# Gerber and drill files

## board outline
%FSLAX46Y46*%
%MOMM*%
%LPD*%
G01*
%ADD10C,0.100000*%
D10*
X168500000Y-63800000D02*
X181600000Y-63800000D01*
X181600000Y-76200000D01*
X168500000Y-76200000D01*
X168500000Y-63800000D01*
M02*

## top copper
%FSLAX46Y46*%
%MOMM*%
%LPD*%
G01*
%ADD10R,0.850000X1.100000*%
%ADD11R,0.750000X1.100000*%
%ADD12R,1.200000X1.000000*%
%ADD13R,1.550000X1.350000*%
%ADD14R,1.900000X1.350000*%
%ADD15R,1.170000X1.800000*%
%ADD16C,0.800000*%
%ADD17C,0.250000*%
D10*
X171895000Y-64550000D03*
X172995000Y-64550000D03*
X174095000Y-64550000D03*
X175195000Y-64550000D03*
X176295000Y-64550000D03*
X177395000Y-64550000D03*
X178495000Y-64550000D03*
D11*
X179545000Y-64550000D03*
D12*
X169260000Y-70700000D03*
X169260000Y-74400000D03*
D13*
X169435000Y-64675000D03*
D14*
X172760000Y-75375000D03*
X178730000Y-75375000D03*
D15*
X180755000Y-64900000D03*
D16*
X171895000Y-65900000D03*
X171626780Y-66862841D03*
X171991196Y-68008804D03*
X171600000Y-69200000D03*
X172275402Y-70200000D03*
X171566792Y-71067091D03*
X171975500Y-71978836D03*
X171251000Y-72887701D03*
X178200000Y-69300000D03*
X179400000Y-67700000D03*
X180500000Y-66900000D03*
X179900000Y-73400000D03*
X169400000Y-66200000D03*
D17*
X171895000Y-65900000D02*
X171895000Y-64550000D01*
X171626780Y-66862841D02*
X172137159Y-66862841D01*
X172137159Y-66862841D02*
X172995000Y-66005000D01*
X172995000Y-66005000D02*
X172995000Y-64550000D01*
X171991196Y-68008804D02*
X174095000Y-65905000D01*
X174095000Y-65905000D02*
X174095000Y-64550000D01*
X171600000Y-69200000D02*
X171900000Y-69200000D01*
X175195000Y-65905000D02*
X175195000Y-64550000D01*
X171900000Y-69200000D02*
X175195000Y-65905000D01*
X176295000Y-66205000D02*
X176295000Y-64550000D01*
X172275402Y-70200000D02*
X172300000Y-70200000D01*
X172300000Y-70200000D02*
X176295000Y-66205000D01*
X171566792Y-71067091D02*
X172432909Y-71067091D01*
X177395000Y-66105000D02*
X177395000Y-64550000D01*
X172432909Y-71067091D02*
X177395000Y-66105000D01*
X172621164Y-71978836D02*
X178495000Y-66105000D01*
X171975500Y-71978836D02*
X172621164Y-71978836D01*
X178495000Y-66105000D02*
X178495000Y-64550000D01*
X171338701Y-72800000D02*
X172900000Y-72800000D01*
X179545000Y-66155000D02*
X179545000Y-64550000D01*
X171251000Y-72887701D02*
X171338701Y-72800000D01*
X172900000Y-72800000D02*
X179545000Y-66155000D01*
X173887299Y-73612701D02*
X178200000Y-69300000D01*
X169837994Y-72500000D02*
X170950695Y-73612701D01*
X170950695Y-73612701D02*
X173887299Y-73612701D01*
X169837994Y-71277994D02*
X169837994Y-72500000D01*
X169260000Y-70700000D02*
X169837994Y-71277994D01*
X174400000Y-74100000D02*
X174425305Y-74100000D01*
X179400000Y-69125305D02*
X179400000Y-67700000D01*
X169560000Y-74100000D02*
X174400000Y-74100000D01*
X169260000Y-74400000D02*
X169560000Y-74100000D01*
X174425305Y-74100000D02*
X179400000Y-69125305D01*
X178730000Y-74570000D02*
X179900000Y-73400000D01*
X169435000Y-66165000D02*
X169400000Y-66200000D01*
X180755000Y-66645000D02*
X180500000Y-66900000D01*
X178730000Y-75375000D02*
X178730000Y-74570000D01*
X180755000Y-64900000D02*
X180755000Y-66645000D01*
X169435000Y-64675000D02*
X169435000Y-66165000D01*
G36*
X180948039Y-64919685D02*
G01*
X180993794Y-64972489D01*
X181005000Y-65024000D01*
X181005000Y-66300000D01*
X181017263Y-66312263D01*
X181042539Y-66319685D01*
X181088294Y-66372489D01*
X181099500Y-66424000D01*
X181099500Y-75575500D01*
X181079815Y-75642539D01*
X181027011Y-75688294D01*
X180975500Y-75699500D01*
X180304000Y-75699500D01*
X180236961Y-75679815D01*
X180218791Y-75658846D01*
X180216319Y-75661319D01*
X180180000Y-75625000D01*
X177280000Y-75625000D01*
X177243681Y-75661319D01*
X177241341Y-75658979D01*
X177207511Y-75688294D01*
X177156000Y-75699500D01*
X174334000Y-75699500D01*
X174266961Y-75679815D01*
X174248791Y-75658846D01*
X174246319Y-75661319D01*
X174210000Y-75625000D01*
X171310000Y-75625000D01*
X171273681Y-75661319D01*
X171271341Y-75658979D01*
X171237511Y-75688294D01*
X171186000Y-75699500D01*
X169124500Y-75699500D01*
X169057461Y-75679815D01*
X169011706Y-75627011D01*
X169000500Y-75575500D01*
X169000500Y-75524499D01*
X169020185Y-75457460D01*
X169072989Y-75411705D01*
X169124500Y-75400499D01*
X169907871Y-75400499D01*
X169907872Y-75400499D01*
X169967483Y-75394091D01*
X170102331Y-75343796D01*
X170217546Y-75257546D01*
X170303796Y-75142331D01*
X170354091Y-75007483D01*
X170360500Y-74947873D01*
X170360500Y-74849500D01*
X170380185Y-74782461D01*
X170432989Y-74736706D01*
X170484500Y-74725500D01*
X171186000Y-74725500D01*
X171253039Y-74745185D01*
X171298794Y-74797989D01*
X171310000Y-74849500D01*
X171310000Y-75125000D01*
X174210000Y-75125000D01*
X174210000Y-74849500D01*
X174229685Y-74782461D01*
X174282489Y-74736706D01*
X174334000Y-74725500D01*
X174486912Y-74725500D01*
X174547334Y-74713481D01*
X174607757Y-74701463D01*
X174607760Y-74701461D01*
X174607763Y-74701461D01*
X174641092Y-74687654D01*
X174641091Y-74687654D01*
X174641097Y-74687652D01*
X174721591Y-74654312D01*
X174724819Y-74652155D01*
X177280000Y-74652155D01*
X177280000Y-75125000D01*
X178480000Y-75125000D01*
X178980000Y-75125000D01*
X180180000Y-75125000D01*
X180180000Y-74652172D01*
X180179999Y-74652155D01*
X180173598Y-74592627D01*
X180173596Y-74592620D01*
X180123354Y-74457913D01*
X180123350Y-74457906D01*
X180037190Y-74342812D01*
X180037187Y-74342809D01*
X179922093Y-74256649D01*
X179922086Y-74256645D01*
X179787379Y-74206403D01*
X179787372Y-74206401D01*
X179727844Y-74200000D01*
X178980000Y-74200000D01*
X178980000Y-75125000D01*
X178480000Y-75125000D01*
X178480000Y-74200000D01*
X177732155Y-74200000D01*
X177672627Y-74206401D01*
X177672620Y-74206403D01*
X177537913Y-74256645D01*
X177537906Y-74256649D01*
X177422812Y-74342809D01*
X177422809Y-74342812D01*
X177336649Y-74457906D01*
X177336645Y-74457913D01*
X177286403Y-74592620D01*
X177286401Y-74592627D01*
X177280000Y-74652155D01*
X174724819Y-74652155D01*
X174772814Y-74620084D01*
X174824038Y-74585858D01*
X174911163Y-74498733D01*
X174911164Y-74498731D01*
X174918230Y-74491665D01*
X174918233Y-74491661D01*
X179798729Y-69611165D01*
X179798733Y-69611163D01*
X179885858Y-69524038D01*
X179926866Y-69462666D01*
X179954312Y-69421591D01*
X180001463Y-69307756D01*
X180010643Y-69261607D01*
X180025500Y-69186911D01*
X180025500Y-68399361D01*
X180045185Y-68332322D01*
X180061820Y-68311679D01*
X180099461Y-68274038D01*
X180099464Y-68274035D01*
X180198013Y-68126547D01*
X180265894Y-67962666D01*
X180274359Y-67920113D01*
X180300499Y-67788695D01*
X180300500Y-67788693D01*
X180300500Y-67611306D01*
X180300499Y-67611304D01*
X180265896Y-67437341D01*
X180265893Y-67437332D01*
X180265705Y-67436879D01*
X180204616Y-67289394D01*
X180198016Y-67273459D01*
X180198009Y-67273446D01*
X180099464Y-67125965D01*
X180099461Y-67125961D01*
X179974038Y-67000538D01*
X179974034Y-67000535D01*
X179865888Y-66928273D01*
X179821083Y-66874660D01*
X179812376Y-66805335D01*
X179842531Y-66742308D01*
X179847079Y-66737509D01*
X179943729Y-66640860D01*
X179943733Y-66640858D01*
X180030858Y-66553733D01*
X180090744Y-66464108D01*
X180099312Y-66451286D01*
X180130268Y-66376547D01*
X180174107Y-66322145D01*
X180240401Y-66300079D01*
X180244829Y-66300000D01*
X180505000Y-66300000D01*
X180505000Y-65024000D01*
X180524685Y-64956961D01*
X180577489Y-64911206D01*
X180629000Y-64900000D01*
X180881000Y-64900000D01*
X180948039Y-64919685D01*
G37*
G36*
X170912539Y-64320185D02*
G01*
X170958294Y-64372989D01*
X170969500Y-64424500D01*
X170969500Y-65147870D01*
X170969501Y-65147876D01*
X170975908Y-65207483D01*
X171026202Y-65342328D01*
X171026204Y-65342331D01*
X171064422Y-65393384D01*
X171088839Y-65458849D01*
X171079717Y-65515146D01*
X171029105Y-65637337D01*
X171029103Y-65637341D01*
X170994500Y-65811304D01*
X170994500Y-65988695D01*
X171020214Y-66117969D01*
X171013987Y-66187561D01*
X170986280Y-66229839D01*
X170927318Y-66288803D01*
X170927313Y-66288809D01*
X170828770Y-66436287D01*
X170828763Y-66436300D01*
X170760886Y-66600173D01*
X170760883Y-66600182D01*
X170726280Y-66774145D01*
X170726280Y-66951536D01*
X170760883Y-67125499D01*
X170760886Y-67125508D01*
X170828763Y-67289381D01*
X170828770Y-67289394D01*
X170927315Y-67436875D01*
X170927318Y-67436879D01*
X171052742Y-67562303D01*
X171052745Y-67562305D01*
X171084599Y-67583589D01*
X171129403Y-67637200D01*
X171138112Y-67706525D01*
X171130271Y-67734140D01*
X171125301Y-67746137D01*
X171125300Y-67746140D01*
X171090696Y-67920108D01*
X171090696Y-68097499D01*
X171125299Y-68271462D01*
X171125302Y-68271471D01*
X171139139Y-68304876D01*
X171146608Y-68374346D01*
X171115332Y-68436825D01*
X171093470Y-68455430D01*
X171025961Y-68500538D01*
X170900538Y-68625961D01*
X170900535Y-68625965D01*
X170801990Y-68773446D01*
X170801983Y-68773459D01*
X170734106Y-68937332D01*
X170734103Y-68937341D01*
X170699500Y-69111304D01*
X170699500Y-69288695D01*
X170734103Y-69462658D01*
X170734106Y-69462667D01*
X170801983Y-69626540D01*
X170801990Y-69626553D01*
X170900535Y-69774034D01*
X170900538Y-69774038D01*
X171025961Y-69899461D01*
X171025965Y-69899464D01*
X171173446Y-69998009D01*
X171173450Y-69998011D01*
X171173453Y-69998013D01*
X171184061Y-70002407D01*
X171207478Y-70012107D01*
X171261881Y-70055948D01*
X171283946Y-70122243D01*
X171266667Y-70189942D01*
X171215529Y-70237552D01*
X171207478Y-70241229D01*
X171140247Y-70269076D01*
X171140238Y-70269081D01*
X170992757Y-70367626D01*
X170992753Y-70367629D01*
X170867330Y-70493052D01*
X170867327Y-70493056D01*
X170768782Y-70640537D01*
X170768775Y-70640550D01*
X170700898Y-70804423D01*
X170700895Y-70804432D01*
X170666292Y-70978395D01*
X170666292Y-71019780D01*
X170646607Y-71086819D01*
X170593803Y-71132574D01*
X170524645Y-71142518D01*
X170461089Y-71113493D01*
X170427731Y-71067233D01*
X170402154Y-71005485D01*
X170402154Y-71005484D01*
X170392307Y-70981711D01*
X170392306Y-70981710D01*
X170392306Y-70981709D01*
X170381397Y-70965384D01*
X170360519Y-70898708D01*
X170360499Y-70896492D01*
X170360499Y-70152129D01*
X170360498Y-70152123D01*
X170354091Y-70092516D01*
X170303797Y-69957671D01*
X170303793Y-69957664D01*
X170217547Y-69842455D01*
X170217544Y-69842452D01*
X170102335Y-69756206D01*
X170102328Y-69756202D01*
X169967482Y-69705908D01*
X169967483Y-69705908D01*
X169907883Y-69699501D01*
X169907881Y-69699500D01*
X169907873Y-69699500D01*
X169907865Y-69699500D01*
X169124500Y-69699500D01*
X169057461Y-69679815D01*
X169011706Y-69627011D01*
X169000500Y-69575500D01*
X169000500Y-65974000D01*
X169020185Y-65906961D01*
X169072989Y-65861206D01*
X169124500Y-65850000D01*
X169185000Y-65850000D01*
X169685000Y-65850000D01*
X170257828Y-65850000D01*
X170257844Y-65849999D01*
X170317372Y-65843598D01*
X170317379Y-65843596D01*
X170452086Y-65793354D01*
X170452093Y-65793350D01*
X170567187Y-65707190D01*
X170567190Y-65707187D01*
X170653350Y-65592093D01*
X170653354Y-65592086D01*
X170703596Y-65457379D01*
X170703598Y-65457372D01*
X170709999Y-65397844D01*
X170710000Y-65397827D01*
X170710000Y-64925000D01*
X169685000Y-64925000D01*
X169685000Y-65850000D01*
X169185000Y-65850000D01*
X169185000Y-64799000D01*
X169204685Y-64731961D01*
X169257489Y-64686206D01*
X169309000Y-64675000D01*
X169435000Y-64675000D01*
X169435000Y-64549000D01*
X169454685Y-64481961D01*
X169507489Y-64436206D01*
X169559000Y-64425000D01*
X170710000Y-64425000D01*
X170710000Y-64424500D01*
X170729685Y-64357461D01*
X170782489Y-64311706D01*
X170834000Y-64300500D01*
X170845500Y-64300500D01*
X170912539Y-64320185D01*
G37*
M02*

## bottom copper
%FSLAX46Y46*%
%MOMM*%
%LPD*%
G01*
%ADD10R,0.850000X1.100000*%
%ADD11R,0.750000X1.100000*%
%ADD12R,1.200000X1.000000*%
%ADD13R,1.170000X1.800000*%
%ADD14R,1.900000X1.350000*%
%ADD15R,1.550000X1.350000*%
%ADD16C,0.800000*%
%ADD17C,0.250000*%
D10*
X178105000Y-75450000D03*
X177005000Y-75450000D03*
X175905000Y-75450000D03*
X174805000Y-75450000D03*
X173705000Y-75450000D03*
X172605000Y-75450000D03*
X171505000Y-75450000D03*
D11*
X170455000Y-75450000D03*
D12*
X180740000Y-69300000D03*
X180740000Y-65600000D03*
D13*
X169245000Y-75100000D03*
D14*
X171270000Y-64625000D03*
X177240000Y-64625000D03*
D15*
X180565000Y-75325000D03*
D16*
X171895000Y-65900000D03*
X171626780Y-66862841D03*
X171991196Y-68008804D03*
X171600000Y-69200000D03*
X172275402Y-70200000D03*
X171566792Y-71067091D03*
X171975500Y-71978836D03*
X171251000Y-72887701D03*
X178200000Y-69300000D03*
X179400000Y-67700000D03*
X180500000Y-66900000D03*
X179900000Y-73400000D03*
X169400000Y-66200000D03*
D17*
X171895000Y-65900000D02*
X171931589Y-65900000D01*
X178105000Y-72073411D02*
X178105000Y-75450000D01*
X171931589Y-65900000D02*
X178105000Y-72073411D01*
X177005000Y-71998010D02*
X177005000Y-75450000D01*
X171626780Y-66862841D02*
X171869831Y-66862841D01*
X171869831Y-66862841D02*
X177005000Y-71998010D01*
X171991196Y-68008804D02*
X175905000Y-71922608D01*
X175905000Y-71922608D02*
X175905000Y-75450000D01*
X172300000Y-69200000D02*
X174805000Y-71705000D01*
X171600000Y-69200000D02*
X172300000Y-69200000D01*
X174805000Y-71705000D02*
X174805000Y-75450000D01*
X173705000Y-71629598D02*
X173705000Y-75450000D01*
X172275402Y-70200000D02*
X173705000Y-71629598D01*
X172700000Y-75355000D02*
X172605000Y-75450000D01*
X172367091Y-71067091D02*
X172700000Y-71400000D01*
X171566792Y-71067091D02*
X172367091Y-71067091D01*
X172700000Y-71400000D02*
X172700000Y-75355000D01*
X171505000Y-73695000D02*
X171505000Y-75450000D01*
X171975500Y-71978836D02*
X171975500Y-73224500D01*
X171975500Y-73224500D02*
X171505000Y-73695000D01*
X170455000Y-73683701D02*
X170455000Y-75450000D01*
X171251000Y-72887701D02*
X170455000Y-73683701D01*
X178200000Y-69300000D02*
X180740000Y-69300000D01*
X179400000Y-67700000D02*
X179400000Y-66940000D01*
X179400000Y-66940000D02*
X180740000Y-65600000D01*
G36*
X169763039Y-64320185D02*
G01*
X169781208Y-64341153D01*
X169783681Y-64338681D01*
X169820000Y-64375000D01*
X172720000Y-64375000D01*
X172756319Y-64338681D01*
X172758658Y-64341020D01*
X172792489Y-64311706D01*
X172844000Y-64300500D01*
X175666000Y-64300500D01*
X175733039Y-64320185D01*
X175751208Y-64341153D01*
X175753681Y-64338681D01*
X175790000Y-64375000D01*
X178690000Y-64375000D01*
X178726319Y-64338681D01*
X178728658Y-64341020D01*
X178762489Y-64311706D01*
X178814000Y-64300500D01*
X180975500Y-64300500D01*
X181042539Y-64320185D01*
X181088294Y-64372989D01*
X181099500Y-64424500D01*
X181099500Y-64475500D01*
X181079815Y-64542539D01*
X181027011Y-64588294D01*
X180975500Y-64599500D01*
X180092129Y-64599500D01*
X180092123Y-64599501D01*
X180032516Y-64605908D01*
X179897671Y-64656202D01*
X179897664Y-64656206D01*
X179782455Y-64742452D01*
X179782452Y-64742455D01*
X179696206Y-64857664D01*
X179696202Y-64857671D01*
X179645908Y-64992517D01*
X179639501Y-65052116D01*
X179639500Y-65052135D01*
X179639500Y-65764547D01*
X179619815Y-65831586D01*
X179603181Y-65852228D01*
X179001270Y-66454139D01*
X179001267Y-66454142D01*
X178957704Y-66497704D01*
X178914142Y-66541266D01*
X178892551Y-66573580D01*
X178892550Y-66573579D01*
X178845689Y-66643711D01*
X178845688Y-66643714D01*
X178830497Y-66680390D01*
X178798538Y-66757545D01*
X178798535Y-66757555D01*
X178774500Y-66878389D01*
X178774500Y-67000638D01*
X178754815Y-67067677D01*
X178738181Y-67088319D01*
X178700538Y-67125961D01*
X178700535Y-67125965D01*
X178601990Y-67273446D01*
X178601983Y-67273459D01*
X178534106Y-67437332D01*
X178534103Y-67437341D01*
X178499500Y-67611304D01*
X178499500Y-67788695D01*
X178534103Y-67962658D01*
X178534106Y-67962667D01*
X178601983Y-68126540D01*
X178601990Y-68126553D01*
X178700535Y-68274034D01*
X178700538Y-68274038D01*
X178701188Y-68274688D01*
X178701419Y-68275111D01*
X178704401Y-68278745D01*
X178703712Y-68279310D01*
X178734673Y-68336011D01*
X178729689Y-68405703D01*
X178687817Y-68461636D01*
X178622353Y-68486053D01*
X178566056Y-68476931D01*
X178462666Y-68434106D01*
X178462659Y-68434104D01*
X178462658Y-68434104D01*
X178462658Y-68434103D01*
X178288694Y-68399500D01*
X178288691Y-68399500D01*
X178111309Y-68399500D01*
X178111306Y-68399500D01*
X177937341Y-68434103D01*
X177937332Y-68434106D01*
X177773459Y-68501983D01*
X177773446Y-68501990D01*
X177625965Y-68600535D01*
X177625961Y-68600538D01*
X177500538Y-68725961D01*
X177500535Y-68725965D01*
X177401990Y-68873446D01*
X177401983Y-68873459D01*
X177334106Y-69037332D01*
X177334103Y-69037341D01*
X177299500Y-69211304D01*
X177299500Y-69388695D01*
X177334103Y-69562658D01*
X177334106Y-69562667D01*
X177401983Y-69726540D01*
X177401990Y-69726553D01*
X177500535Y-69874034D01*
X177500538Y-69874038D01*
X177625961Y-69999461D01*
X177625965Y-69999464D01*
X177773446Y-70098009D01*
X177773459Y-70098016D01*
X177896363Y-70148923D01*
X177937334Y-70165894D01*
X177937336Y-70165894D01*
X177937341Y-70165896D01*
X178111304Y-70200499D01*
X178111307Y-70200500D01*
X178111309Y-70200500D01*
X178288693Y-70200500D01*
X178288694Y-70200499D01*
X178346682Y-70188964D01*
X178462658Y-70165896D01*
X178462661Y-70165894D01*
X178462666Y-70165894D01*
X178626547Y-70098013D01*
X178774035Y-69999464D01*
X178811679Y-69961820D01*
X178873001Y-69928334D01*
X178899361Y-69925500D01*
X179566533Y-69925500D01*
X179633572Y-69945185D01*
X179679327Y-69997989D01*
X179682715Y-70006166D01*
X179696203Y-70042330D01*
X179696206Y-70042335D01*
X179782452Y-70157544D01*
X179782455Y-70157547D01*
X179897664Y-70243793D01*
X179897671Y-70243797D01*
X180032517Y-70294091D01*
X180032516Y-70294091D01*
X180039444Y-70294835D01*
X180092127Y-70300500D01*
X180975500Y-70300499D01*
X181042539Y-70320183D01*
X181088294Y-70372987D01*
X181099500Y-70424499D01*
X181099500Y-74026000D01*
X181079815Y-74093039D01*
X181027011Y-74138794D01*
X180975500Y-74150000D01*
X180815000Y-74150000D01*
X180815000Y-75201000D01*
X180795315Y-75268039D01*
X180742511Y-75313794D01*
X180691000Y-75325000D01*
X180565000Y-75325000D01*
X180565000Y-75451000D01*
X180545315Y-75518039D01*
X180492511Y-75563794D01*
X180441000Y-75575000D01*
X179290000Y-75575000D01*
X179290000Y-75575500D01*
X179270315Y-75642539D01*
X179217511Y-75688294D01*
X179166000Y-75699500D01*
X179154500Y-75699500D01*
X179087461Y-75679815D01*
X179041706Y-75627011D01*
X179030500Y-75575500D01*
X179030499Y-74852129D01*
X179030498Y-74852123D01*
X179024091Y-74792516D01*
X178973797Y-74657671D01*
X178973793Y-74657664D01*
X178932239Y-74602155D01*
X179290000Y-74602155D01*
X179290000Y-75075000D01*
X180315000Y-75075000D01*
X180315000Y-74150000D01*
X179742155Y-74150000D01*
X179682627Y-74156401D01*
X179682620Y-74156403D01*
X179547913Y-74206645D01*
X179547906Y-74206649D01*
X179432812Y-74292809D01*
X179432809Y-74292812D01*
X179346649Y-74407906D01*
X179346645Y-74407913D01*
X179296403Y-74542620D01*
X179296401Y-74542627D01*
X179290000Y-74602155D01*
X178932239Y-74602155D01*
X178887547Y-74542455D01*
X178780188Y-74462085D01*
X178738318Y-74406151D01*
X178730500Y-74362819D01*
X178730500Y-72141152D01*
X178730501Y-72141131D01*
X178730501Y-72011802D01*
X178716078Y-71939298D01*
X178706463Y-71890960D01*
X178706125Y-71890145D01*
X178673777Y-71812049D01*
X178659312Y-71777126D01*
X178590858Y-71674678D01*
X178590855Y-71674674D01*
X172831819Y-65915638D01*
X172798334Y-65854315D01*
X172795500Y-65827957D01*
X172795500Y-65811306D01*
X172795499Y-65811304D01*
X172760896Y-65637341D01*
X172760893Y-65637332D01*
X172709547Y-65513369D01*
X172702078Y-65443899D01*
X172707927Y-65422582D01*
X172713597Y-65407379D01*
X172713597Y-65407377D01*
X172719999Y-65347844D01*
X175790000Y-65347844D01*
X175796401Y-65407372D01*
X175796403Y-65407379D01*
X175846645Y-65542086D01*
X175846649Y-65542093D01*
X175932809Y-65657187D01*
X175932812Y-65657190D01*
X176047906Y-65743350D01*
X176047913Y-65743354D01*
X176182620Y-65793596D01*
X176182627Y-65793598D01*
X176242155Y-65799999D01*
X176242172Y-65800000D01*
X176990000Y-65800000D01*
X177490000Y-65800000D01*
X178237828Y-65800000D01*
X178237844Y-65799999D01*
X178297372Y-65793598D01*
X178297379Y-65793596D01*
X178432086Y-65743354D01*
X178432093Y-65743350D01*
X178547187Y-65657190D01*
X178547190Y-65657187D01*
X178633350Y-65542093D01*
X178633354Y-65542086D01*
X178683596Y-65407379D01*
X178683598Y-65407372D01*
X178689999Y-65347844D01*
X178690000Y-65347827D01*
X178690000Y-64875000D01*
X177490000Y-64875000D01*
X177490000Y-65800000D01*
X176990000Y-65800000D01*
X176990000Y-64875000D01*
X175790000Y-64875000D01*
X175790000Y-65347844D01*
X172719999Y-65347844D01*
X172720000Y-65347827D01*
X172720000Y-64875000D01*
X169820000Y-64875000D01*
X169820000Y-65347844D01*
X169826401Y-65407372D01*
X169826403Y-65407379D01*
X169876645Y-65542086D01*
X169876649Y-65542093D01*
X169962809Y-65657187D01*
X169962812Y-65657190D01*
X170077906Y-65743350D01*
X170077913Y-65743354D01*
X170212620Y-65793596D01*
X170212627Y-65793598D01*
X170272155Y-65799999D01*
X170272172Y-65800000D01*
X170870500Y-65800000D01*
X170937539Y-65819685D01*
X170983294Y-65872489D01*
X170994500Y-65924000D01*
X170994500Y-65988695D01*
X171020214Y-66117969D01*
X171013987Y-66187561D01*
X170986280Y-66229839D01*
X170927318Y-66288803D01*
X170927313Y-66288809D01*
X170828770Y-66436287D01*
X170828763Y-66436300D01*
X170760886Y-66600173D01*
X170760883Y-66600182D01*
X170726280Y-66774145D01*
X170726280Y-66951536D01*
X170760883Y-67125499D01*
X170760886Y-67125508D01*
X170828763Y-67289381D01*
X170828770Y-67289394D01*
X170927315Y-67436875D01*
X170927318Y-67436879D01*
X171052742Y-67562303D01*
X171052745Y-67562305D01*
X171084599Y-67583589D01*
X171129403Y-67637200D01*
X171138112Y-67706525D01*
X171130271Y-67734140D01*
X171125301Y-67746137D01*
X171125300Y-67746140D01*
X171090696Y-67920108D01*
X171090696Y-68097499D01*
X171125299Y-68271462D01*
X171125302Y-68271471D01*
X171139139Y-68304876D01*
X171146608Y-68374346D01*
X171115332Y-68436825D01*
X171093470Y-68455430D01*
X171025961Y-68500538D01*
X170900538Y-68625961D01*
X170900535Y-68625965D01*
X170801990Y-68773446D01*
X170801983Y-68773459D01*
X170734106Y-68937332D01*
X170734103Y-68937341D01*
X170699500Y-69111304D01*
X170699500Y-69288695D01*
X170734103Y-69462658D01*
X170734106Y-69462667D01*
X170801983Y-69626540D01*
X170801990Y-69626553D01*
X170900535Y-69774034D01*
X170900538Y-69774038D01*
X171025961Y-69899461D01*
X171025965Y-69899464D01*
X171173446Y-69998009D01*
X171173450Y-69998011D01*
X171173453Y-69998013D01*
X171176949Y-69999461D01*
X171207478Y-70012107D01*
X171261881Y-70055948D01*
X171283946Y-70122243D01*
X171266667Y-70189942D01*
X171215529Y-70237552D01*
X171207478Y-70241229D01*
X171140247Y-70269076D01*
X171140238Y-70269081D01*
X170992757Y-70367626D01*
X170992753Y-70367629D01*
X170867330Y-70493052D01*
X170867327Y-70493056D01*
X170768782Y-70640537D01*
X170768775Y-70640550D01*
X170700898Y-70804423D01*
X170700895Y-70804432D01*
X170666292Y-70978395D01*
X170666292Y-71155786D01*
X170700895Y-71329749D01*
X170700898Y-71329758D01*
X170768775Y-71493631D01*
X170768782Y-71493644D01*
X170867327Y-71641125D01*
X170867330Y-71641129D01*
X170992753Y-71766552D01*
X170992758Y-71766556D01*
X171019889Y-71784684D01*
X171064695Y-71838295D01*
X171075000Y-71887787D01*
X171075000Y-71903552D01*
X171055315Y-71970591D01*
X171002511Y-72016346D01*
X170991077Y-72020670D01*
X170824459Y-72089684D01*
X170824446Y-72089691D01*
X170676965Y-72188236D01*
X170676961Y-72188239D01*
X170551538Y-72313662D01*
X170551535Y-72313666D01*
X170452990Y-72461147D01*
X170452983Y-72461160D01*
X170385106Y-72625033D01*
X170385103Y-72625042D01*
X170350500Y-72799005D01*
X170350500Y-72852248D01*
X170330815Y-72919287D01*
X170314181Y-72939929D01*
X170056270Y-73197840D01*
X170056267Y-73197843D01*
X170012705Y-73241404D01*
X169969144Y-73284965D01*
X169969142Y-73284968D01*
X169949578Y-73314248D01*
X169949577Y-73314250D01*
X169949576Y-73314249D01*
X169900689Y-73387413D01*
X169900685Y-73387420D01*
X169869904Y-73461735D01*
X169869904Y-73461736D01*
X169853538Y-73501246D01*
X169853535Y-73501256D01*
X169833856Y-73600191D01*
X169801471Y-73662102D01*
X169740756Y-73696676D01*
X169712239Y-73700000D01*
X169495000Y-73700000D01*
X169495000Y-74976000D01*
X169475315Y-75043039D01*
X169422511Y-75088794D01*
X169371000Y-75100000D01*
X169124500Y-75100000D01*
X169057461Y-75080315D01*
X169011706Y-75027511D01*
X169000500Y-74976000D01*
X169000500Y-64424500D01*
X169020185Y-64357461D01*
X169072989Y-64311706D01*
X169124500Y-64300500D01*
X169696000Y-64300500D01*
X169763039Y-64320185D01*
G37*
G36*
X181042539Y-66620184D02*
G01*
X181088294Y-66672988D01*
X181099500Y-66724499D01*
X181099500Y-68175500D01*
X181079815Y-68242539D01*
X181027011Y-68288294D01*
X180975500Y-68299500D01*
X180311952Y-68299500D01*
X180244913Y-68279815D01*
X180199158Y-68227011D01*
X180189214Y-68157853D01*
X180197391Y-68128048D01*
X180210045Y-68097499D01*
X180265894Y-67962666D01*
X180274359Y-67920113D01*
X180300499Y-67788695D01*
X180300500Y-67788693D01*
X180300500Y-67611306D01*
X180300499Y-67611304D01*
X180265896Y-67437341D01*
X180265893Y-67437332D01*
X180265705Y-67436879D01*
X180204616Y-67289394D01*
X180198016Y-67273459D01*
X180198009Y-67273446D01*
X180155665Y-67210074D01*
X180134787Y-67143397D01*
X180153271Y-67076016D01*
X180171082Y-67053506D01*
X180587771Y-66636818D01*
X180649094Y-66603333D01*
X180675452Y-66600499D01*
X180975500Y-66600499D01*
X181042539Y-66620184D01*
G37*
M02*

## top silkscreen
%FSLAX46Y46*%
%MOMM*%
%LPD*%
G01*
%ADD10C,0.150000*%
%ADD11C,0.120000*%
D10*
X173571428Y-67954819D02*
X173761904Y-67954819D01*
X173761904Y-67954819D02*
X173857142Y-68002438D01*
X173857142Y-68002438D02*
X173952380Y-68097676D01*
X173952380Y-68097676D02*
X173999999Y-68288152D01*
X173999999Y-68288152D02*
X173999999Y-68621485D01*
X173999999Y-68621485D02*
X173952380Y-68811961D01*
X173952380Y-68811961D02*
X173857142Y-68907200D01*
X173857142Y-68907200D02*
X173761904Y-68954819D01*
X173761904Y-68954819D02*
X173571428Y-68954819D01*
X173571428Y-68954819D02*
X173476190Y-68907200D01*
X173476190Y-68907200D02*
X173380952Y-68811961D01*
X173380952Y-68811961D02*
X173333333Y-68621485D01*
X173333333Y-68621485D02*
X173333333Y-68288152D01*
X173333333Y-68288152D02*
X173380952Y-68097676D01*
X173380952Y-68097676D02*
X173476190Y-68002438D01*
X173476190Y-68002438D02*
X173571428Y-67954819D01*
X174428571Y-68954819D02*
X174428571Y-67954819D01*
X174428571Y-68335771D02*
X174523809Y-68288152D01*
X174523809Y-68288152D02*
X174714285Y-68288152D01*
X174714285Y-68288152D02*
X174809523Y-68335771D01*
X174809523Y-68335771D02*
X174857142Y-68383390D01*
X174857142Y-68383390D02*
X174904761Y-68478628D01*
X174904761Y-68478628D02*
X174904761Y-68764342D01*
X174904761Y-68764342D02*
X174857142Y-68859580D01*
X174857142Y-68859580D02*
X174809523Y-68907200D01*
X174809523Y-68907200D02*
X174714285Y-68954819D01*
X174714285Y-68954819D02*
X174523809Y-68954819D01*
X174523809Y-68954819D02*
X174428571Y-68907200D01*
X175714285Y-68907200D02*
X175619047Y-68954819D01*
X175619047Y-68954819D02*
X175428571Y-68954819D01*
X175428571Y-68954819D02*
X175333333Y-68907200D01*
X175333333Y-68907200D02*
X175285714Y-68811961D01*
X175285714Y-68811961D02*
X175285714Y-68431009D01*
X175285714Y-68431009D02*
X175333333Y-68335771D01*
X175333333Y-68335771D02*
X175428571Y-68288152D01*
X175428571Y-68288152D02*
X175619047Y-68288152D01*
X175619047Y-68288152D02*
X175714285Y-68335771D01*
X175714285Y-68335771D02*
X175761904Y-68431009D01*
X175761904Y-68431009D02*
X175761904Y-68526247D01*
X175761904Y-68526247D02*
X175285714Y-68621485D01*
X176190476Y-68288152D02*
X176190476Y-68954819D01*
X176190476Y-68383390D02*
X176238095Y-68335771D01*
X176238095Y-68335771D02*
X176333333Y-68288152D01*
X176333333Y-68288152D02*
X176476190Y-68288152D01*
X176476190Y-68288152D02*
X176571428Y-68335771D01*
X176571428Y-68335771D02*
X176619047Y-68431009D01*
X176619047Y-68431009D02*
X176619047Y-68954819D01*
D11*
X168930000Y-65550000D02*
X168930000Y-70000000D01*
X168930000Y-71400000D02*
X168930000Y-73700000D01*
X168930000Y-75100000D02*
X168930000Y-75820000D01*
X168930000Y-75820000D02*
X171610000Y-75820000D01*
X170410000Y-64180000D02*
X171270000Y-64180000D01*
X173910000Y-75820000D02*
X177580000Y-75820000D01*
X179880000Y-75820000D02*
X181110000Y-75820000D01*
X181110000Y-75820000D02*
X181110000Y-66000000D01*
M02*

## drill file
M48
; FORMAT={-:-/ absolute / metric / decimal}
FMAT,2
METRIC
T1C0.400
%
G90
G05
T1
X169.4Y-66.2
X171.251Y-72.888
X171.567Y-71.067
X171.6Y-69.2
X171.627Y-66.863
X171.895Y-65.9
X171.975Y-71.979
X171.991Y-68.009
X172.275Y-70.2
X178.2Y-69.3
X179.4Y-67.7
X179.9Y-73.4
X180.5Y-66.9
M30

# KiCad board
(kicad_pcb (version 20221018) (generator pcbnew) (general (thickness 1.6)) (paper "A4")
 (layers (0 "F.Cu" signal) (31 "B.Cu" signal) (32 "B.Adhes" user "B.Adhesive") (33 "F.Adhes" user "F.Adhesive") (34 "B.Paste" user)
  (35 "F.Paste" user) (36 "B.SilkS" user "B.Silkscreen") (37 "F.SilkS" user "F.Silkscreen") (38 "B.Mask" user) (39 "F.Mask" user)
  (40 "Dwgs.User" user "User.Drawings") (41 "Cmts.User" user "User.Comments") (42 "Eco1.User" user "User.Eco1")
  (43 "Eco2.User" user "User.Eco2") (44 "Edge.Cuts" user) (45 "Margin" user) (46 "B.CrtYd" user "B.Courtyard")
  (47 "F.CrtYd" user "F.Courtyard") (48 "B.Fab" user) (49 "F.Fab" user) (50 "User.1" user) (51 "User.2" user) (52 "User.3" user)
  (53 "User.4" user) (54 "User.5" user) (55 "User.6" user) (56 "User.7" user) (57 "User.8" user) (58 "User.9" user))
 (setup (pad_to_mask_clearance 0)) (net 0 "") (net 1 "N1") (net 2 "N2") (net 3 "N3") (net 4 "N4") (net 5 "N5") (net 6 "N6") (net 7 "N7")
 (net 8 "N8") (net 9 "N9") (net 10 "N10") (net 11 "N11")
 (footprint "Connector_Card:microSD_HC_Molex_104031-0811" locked (layer "F.Cu") (at 175 70)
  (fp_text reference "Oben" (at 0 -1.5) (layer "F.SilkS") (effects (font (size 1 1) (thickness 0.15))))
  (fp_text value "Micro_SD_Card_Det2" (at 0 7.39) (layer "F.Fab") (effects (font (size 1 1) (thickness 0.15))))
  (fp_line (start -6.07 -4.45) (end -6.07 0) (stroke (width 0.12) (type solid)) (layer "F.SilkS"))
  (fp_line (start -6.07 1.4) (end -6.07 3.7) (stroke (width 0.12) (type solid)) (layer "F.SilkS"))
  (fp_line (start -6.07 5.1) (end -6.07 5.82) (stroke (width 0.12) (type solid)) (layer "F.SilkS"))
  (fp_line (start -6.07 5.82) (end -3.39 5.82) (stroke (width 0.12) (type solid)) (layer "F.SilkS"))
  (fp_line (start -4.59 -5.82) (end -3.73 -5.82) (stroke (width 0.12) (type solid)) (layer "F.SilkS"))
  (fp_line (start -1.09 5.82) (end 2.58 5.82) (stroke (width 0.12) (type solid)) (layer "F.SilkS"))
  (fp_line (start 4.88 5.82) (end 6.11 5.82) (stroke (width 0.12) (type solid)) (layer "F.SilkS"))
  (fp_line (start 6.11 5.82) (end 6.11 -4) (stroke (width 0.12) (type solid)) (layer "F.SilkS"))
  (pad "1" smd rect locked (at -3.105 -5.45) (size 0.85 1.1) (layers "F.Cu" "F.Paste" "F.Mask") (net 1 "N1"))
  (pad "2" smd rect locked (at -2.005 -5.45) (size 0.85 1.1) (layers "F.Cu" "F.Paste" "F.Mask") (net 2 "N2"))
  (pad "3" smd rect locked (at -0.905 -5.45) (size 0.85 1.1) (layers "F.Cu" "F.Paste" "F.Mask") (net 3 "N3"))
  (pad "4" smd rect locked (at 0.195 -5.45) (size 0.85 1.1) (layers "F.Cu" "F.Paste" "F.Mask") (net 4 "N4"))
  (pad "5" smd rect locked (at 1.295 -5.45) (size 0.85 1.1) (layers "F.Cu" "F.Paste" "F.Mask") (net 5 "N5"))
  (pad "6" smd rect locked (at 2.395 -5.45) (size 0.85 1.1) (layers "F.Cu" "F.Paste" "F.Mask") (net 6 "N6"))
  (pad "7" smd rect locked (at 3.495 -5.45) (size 0.85 1.1) (layers "F.Cu" "F.Paste" "F.Mask") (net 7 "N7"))
  (pad "8" smd rect locked (at 4.545 -5.45) (size 0.75 1.1) (layers "F.Cu" "F.Paste" "F.Mask") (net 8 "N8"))
  (pad "9" smd rect locked (at -5.74 0.7) (size 1.2 1) (layers "F.Cu" "F.Paste" "F.Mask") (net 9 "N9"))
  (pad "10" smd rect locked (at -5.74 4.4) (size 1.2 1) (layers "F.Cu" "F.Paste" "F.Mask") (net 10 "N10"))
  (pad "11" smd rect locked (at -5.565 -5.325) (size 1.55 1.35) (layers "F.Cu" "F.Paste" "F.Mask") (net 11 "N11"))
  (pad "11" smd rect locked (at -2.24 5.375) (size 1.9 1.35) (layers "F.Cu" "F.Paste" "F.Mask") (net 11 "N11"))
  (pad "11" smd rect locked (at 3.73 5.375) (size 1.9 1.35) (layers "F.Cu" "F.Paste" "F.Mask") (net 11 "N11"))
  (pad "11" smd rect locked (at 5.755 -5.1) (size 1.17 1.8) (layers "F.Cu" "F.Paste" "F.Mask") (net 11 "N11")))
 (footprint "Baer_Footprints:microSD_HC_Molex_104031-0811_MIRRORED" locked (layer "B.Cu") (at 175 70)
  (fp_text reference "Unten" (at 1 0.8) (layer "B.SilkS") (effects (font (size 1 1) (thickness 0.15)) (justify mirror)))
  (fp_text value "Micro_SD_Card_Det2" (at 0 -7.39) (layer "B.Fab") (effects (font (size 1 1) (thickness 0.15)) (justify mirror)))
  (pad "1" smd rect locked (at 3.105 5.45) (size 0.85 1.1) (layers "B.Cu" "B.Paste" "B.Mask") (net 1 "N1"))
  (pad "2" smd rect locked (at 2.005 5.45) (size 0.85 1.1) (layers "B.Cu" "B.Paste" "B.Mask") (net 2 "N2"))
  (pad "3" smd rect locked (at 0.905 5.45) (size 0.85 1.1) (layers "B.Cu" "B.Paste" "B.Mask") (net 3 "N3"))
  (pad "4" smd rect locked (at -0.195 5.45) (size 0.85 1.1) (layers "B.Cu" "B.Paste" "B.Mask") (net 4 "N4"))
  (pad "5" smd rect locked (at -1.295 5.45) (size 0.85 1.1) (layers "B.Cu" "B.Paste" "B.Mask") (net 5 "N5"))
  (pad "6" smd rect locked (at -2.395 5.45) (size 0.85 1.1) (layers "B.Cu" "B.Paste" "B.Mask") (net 6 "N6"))
  (pad "7" smd rect locked (at -3.495 5.45) (size 0.85 1.1) (layers "B.Cu" "B.Paste" "B.Mask") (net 7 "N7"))
  (pad "8" smd rect locked (at -4.545 5.45) (size 0.75 1.1) (layers "B.Cu" "B.Paste" "B.Mask") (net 8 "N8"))
  (pad "9" smd rect locked (at 5.74 -0.7) (size 1.2 1) (layers "B.Cu" "B.Paste" "B.Mask") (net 9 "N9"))
  (pad "10" smd rect locked (at 5.74 -4.4) (size 1.2 1) (layers "B.Cu" "B.Paste" "B.Mask") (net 10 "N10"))
  (pad "11" smd rect locked (at -5.755 5.1) (size 1.17 1.8) (layers "B.Cu" "B.Paste" "B.Mask") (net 11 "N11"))
  (pad "11" smd rect locked (at -3.73 -5.375) (size 1.9 1.35) (layers "B.Cu" "B.Paste" "B.Mask") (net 11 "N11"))
  (pad "11" smd rect locked (at 2.24 -5.375) (size 1.9 1.35) (layers "B.Cu" "B.Paste" "B.Mask") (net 11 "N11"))
  (pad "11" smd rect locked (at 5.565 5.325) (size 1.55 1.35) (layers "B.Cu" "B.Paste" "B.Mask") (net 11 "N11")))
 (gr_rect (start 168.5 63.8) (end 181.6 76.2) (stroke (width 0.1) (type default)) (fill none) (layer "Edge.Cuts"))
 (segment (start 171.895 65.9) (end 171.895 64.55) (width 0.25) (layer "F.Cu") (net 1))
 (via (at 171.895 65.9) (size 0.8) (drill 0.4) (layers "F.Cu" "B.Cu") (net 1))
 (segment (start 171.895 65.9) (end 171.931589 65.9) (width 0.25) (layer "B.Cu") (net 1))
 (segment (start 178.105 72.073411) (end 178.105 75.45) (width 0.25) (layer "B.Cu") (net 1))
 (segment (start 171.931589 65.9) (end 178.105 72.073411) (width 0.25) (layer "B.Cu") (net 1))
 (segment (start 171.62678 66.862841) (end 172.137159 66.862841) (width 0.25) (layer "F.Cu") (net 2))
 (segment (start 172.137159 66.862841) (end 172.995 66.005) (width 0.25) (layer "F.Cu") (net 2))
 (segment (start 172.995 66.005) (end 172.995 64.55) (width 0.25) (layer "F.Cu") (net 2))
 (via (at 171.62678 66.862841) (size 0.8) (drill 0.4) (layers "F.Cu" "B.Cu") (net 2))
 (segment (start 177.005 71.99801) (end 177.005 75.45) (width 0.25) (layer "B.Cu") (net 2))
 (segment (start 171.62678 66.862841) (end 171.869831 66.862841) (width 0.25) (layer "B.Cu") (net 2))
 (segment (start 171.869831 66.862841) (end 177.005 71.99801) (width 0.25) (layer "B.Cu") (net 2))
 (segment (start 171.991196 68.008804) (end 174.095 65.905) (width 0.25) (layer "F.Cu") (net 3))
 (segment (start 174.095 65.905) (end 174.095 64.55) (width 0.25) (layer "F.Cu") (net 3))
 (via (at 171.991196 68.008804) (size 0.8) (drill 0.4) (layers "F.Cu" "B.Cu") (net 3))
 (segment (start 171.991196 68.008804) (end 175.905 71.922608) (width 0.25) (layer "B.Cu") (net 3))
 (segment (start 175.905 71.922608) (end 175.905 75.45) (width 0.25) (layer "B.Cu") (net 3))
 (segment (start 171.6 69.2) (end 171.9 69.2) (width 0.25) (layer "F.Cu") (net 4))
 (segment (start 175.195 65.905) (end 175.195 64.55) (width 0.25) (layer "F.Cu") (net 4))
 (segment (start 171.9 69.2) (end 175.195 65.905) (width 0.25) (layer "F.Cu") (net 4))
 (via (at 171.6 69.2) (size 0.8) (drill 0.4) (layers "F.Cu" "B.Cu") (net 4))
 (segment (start 172.3 69.2) (end 174.805 71.705) (width 0.25) (layer "B.Cu") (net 4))
 (segment (start 171.6 69.2) (end 172.3 69.2) (width 0.25) (layer "B.Cu") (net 4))
 (segment (start 174.805 71.705) (end 174.805 75.45) (width 0.25) (layer "B.Cu") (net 4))
 (segment (start 176.295 66.205) (end 176.295 64.55) (width 0.25) (layer "F.Cu") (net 5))
 (segment (start 172.275402 70.2) (end 172.3 70.2) (width 0.25) (layer "F.Cu") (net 5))
 (segment (start 172.3 70.2) (end 176.295 66.205) (width 0.25) (layer "F.Cu") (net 5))
 (via (at 172.275402 70.2) (size 0.8) (drill 0.4) (layers "F.Cu" "B.Cu") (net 5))
 (segment (start 173.705 71.629598) (end 173.705 75.45) (width 0.25) (layer "B.Cu") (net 5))
 (segment (start 172.275402 70.2) (end 173.705 71.629598) (width 0.25) (layer "B.Cu") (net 5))
 (segment (start 171.566792 71.067091) (end 172.432909 71.067091) (width 0.25) (layer "F.Cu") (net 6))
 (segment (start 177.395 66.105) (end 177.395 64.55) (width 0.25) (layer "F.Cu") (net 6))
 (segment (start 172.432909 71.067091) (end 177.395 66.105) (width 0.25) (layer "F.Cu") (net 6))
 (via (at 171.566792 71.067091) (size 0.8) (drill 0.4) (layers "F.Cu" "B.Cu") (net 6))
 (segment (start 172.7 75.355) (end 172.605 75.45) (width 0.25) (layer "B.Cu") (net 6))
 (segment (start 172.367091 71.067091) (end 172.7 71.4) (width 0.25) (layer "B.Cu") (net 6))
 (segment (start 171.566792 71.067091) (end 172.367091 71.067091) (width 0.25) (layer "B.Cu") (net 6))
 (segment (start 172.7 71.4) (end 172.7 75.355) (width 0.25) (layer "B.Cu") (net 6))
 (segment (start 172.621164 71.978836) (end 178.495 66.105) (width 0.25) (layer "F.Cu") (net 7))
 (segment (start 171.9755 71.978836) (end 172.621164 71.978836) (width 0.25) (layer "F.Cu") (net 7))
 (segment (start 178.495 66.105) (end 178.495 64.55) (width 0.25) (layer "F.Cu") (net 7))
 (via (at 171.9755 71.978836) (size 0.8) (drill 0.4) (layers "F.Cu" "B.Cu") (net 7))
 (segment (start 171.505 73.695) (end 171.505 75.45) (width 0.25) (layer "B.Cu") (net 7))
 (segment (start 171.9755 71.978836) (end 171.9755 73.2245) (width 0.25) (layer "B.Cu") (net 7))
 (segment (start 171.9755 73.2245) (end 171.505 73.695) (width 0.25) (layer "B.Cu") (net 7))
 (segment (start 171.338701 72.8) (end 172.9 72.8) (width 0.25) (layer "F.Cu") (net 8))
 (segment (start 179.545 66.155) (end 179.545 64.55) (width 0.25) (layer "F.Cu") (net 8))
 (segment (start 171.251 72.887701) (end 171.338701 72.8) (width 0.25) (layer "F.Cu") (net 8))
 (segment (start 172.9 72.8) (end 179.545 66.155) (width 0.25) (layer "F.Cu") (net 8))
 (via (at 171.251 72.887701) (size 0.8) (drill 0.4) (layers "F.Cu" "B.Cu") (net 8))
 (segment (start 170.455 73.683701) (end 170.455 75.45) (width 0.25) (layer "B.Cu") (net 8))
 (segment (start 171.251 72.887701) (end 170.455 73.683701) (width 0.25) (layer "B.Cu") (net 8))
 (segment (start 173.887299 73.612701) (end 178.2 69.3) (width 0.25) (layer "F.Cu") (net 9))
 (segment (start 169.837994 72.5) (end 170.950695 73.612701) (width 0.25) (layer "F.Cu") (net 9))
 (segment (start 170.950695 73.612701) (end 173.887299 73.612701) (width 0.25) (layer "F.Cu") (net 9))
 (segment (start 169.837994 71.277994) (end 169.837994 72.5) (width 0.25) (layer "F.Cu") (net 9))
 (segment (start 169.26 70.7) (end 169.837994 71.277994) (width 0.25) (layer "F.Cu") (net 9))
 (via (at 178.2 69.3) (size 0.8) (drill 0.4) (layers "F.Cu" "B.Cu") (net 9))
 (segment (start 178.2 69.3) (end 180.74 69.3) (width 0.25) (layer "B.Cu") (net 9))
 (segment (start 174.4 74.1) (end 174.425305 74.1) (width 0.25) (layer "F.Cu") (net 10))
 (segment (start 179.4 69.125305) (end 179.4 67.7) (width 0.25) (layer "F.Cu") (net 10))
 (segment (start 169.56 74.1) (end 174.4 74.1) (width 0.25) (layer "F.Cu") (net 10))
 (segment (start 169.26 74.4) (end 169.56 74.1) (width 0.25) (layer "F.Cu") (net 10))
 (segment (start 174.425305 74.1) (end 179.4 69.125305) (width 0.25) (layer "F.Cu") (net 10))
 (via (at 179.4 67.7) (size 0.8) (drill 0.4) (layers "F.Cu" "B.Cu") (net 10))
 (segment (start 179.4 67.7) (end 179.4 66.94) (width 0.25) (layer "B.Cu") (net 10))
 (segment (start 179.4 66.94) (end 180.74 65.6) (width 0.25) (layer "B.Cu") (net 10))
 (segment (start 178.73 74.57) (end 179.9 73.4) (width 0.25) (layer "F.Cu") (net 11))
 (segment (start 169.435 66.165) (end 169.4 66.2) (width 0.25) (layer "F.Cu") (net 11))
 (segment (start 180.755 66.645) (end 180.5 66.9) (width 0.25) (layer "F.Cu") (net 11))
 (segment (start 178.73 75.375) (end 178.73 74.57) (width 0.25) (layer "F.Cu") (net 11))
 (segment (start 180.755 64.9) (end 180.755 66.645) (width 0.25) (layer "F.Cu") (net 11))
 (segment (start 169.435 64.675) (end 169.435 66.165) (width 0.25) (layer "F.Cu") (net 11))
 (via (at 180.5 66.9) (size 0.8) (drill 0.4) (layers "F.Cu" "B.Cu") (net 11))
 (via (at 179.9 73.4) (size 0.8) (drill 0.4) (layers "F.Cu" "B.Cu") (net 11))
 (via (at 169.4 66.2) (size 0.8) (drill 0.4) (layers "F.Cu" "B.Cu") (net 11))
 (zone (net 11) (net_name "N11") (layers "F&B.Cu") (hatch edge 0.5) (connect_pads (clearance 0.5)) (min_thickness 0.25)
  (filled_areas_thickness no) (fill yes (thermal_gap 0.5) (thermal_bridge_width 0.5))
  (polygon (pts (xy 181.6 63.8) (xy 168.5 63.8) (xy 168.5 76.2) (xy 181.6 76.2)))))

